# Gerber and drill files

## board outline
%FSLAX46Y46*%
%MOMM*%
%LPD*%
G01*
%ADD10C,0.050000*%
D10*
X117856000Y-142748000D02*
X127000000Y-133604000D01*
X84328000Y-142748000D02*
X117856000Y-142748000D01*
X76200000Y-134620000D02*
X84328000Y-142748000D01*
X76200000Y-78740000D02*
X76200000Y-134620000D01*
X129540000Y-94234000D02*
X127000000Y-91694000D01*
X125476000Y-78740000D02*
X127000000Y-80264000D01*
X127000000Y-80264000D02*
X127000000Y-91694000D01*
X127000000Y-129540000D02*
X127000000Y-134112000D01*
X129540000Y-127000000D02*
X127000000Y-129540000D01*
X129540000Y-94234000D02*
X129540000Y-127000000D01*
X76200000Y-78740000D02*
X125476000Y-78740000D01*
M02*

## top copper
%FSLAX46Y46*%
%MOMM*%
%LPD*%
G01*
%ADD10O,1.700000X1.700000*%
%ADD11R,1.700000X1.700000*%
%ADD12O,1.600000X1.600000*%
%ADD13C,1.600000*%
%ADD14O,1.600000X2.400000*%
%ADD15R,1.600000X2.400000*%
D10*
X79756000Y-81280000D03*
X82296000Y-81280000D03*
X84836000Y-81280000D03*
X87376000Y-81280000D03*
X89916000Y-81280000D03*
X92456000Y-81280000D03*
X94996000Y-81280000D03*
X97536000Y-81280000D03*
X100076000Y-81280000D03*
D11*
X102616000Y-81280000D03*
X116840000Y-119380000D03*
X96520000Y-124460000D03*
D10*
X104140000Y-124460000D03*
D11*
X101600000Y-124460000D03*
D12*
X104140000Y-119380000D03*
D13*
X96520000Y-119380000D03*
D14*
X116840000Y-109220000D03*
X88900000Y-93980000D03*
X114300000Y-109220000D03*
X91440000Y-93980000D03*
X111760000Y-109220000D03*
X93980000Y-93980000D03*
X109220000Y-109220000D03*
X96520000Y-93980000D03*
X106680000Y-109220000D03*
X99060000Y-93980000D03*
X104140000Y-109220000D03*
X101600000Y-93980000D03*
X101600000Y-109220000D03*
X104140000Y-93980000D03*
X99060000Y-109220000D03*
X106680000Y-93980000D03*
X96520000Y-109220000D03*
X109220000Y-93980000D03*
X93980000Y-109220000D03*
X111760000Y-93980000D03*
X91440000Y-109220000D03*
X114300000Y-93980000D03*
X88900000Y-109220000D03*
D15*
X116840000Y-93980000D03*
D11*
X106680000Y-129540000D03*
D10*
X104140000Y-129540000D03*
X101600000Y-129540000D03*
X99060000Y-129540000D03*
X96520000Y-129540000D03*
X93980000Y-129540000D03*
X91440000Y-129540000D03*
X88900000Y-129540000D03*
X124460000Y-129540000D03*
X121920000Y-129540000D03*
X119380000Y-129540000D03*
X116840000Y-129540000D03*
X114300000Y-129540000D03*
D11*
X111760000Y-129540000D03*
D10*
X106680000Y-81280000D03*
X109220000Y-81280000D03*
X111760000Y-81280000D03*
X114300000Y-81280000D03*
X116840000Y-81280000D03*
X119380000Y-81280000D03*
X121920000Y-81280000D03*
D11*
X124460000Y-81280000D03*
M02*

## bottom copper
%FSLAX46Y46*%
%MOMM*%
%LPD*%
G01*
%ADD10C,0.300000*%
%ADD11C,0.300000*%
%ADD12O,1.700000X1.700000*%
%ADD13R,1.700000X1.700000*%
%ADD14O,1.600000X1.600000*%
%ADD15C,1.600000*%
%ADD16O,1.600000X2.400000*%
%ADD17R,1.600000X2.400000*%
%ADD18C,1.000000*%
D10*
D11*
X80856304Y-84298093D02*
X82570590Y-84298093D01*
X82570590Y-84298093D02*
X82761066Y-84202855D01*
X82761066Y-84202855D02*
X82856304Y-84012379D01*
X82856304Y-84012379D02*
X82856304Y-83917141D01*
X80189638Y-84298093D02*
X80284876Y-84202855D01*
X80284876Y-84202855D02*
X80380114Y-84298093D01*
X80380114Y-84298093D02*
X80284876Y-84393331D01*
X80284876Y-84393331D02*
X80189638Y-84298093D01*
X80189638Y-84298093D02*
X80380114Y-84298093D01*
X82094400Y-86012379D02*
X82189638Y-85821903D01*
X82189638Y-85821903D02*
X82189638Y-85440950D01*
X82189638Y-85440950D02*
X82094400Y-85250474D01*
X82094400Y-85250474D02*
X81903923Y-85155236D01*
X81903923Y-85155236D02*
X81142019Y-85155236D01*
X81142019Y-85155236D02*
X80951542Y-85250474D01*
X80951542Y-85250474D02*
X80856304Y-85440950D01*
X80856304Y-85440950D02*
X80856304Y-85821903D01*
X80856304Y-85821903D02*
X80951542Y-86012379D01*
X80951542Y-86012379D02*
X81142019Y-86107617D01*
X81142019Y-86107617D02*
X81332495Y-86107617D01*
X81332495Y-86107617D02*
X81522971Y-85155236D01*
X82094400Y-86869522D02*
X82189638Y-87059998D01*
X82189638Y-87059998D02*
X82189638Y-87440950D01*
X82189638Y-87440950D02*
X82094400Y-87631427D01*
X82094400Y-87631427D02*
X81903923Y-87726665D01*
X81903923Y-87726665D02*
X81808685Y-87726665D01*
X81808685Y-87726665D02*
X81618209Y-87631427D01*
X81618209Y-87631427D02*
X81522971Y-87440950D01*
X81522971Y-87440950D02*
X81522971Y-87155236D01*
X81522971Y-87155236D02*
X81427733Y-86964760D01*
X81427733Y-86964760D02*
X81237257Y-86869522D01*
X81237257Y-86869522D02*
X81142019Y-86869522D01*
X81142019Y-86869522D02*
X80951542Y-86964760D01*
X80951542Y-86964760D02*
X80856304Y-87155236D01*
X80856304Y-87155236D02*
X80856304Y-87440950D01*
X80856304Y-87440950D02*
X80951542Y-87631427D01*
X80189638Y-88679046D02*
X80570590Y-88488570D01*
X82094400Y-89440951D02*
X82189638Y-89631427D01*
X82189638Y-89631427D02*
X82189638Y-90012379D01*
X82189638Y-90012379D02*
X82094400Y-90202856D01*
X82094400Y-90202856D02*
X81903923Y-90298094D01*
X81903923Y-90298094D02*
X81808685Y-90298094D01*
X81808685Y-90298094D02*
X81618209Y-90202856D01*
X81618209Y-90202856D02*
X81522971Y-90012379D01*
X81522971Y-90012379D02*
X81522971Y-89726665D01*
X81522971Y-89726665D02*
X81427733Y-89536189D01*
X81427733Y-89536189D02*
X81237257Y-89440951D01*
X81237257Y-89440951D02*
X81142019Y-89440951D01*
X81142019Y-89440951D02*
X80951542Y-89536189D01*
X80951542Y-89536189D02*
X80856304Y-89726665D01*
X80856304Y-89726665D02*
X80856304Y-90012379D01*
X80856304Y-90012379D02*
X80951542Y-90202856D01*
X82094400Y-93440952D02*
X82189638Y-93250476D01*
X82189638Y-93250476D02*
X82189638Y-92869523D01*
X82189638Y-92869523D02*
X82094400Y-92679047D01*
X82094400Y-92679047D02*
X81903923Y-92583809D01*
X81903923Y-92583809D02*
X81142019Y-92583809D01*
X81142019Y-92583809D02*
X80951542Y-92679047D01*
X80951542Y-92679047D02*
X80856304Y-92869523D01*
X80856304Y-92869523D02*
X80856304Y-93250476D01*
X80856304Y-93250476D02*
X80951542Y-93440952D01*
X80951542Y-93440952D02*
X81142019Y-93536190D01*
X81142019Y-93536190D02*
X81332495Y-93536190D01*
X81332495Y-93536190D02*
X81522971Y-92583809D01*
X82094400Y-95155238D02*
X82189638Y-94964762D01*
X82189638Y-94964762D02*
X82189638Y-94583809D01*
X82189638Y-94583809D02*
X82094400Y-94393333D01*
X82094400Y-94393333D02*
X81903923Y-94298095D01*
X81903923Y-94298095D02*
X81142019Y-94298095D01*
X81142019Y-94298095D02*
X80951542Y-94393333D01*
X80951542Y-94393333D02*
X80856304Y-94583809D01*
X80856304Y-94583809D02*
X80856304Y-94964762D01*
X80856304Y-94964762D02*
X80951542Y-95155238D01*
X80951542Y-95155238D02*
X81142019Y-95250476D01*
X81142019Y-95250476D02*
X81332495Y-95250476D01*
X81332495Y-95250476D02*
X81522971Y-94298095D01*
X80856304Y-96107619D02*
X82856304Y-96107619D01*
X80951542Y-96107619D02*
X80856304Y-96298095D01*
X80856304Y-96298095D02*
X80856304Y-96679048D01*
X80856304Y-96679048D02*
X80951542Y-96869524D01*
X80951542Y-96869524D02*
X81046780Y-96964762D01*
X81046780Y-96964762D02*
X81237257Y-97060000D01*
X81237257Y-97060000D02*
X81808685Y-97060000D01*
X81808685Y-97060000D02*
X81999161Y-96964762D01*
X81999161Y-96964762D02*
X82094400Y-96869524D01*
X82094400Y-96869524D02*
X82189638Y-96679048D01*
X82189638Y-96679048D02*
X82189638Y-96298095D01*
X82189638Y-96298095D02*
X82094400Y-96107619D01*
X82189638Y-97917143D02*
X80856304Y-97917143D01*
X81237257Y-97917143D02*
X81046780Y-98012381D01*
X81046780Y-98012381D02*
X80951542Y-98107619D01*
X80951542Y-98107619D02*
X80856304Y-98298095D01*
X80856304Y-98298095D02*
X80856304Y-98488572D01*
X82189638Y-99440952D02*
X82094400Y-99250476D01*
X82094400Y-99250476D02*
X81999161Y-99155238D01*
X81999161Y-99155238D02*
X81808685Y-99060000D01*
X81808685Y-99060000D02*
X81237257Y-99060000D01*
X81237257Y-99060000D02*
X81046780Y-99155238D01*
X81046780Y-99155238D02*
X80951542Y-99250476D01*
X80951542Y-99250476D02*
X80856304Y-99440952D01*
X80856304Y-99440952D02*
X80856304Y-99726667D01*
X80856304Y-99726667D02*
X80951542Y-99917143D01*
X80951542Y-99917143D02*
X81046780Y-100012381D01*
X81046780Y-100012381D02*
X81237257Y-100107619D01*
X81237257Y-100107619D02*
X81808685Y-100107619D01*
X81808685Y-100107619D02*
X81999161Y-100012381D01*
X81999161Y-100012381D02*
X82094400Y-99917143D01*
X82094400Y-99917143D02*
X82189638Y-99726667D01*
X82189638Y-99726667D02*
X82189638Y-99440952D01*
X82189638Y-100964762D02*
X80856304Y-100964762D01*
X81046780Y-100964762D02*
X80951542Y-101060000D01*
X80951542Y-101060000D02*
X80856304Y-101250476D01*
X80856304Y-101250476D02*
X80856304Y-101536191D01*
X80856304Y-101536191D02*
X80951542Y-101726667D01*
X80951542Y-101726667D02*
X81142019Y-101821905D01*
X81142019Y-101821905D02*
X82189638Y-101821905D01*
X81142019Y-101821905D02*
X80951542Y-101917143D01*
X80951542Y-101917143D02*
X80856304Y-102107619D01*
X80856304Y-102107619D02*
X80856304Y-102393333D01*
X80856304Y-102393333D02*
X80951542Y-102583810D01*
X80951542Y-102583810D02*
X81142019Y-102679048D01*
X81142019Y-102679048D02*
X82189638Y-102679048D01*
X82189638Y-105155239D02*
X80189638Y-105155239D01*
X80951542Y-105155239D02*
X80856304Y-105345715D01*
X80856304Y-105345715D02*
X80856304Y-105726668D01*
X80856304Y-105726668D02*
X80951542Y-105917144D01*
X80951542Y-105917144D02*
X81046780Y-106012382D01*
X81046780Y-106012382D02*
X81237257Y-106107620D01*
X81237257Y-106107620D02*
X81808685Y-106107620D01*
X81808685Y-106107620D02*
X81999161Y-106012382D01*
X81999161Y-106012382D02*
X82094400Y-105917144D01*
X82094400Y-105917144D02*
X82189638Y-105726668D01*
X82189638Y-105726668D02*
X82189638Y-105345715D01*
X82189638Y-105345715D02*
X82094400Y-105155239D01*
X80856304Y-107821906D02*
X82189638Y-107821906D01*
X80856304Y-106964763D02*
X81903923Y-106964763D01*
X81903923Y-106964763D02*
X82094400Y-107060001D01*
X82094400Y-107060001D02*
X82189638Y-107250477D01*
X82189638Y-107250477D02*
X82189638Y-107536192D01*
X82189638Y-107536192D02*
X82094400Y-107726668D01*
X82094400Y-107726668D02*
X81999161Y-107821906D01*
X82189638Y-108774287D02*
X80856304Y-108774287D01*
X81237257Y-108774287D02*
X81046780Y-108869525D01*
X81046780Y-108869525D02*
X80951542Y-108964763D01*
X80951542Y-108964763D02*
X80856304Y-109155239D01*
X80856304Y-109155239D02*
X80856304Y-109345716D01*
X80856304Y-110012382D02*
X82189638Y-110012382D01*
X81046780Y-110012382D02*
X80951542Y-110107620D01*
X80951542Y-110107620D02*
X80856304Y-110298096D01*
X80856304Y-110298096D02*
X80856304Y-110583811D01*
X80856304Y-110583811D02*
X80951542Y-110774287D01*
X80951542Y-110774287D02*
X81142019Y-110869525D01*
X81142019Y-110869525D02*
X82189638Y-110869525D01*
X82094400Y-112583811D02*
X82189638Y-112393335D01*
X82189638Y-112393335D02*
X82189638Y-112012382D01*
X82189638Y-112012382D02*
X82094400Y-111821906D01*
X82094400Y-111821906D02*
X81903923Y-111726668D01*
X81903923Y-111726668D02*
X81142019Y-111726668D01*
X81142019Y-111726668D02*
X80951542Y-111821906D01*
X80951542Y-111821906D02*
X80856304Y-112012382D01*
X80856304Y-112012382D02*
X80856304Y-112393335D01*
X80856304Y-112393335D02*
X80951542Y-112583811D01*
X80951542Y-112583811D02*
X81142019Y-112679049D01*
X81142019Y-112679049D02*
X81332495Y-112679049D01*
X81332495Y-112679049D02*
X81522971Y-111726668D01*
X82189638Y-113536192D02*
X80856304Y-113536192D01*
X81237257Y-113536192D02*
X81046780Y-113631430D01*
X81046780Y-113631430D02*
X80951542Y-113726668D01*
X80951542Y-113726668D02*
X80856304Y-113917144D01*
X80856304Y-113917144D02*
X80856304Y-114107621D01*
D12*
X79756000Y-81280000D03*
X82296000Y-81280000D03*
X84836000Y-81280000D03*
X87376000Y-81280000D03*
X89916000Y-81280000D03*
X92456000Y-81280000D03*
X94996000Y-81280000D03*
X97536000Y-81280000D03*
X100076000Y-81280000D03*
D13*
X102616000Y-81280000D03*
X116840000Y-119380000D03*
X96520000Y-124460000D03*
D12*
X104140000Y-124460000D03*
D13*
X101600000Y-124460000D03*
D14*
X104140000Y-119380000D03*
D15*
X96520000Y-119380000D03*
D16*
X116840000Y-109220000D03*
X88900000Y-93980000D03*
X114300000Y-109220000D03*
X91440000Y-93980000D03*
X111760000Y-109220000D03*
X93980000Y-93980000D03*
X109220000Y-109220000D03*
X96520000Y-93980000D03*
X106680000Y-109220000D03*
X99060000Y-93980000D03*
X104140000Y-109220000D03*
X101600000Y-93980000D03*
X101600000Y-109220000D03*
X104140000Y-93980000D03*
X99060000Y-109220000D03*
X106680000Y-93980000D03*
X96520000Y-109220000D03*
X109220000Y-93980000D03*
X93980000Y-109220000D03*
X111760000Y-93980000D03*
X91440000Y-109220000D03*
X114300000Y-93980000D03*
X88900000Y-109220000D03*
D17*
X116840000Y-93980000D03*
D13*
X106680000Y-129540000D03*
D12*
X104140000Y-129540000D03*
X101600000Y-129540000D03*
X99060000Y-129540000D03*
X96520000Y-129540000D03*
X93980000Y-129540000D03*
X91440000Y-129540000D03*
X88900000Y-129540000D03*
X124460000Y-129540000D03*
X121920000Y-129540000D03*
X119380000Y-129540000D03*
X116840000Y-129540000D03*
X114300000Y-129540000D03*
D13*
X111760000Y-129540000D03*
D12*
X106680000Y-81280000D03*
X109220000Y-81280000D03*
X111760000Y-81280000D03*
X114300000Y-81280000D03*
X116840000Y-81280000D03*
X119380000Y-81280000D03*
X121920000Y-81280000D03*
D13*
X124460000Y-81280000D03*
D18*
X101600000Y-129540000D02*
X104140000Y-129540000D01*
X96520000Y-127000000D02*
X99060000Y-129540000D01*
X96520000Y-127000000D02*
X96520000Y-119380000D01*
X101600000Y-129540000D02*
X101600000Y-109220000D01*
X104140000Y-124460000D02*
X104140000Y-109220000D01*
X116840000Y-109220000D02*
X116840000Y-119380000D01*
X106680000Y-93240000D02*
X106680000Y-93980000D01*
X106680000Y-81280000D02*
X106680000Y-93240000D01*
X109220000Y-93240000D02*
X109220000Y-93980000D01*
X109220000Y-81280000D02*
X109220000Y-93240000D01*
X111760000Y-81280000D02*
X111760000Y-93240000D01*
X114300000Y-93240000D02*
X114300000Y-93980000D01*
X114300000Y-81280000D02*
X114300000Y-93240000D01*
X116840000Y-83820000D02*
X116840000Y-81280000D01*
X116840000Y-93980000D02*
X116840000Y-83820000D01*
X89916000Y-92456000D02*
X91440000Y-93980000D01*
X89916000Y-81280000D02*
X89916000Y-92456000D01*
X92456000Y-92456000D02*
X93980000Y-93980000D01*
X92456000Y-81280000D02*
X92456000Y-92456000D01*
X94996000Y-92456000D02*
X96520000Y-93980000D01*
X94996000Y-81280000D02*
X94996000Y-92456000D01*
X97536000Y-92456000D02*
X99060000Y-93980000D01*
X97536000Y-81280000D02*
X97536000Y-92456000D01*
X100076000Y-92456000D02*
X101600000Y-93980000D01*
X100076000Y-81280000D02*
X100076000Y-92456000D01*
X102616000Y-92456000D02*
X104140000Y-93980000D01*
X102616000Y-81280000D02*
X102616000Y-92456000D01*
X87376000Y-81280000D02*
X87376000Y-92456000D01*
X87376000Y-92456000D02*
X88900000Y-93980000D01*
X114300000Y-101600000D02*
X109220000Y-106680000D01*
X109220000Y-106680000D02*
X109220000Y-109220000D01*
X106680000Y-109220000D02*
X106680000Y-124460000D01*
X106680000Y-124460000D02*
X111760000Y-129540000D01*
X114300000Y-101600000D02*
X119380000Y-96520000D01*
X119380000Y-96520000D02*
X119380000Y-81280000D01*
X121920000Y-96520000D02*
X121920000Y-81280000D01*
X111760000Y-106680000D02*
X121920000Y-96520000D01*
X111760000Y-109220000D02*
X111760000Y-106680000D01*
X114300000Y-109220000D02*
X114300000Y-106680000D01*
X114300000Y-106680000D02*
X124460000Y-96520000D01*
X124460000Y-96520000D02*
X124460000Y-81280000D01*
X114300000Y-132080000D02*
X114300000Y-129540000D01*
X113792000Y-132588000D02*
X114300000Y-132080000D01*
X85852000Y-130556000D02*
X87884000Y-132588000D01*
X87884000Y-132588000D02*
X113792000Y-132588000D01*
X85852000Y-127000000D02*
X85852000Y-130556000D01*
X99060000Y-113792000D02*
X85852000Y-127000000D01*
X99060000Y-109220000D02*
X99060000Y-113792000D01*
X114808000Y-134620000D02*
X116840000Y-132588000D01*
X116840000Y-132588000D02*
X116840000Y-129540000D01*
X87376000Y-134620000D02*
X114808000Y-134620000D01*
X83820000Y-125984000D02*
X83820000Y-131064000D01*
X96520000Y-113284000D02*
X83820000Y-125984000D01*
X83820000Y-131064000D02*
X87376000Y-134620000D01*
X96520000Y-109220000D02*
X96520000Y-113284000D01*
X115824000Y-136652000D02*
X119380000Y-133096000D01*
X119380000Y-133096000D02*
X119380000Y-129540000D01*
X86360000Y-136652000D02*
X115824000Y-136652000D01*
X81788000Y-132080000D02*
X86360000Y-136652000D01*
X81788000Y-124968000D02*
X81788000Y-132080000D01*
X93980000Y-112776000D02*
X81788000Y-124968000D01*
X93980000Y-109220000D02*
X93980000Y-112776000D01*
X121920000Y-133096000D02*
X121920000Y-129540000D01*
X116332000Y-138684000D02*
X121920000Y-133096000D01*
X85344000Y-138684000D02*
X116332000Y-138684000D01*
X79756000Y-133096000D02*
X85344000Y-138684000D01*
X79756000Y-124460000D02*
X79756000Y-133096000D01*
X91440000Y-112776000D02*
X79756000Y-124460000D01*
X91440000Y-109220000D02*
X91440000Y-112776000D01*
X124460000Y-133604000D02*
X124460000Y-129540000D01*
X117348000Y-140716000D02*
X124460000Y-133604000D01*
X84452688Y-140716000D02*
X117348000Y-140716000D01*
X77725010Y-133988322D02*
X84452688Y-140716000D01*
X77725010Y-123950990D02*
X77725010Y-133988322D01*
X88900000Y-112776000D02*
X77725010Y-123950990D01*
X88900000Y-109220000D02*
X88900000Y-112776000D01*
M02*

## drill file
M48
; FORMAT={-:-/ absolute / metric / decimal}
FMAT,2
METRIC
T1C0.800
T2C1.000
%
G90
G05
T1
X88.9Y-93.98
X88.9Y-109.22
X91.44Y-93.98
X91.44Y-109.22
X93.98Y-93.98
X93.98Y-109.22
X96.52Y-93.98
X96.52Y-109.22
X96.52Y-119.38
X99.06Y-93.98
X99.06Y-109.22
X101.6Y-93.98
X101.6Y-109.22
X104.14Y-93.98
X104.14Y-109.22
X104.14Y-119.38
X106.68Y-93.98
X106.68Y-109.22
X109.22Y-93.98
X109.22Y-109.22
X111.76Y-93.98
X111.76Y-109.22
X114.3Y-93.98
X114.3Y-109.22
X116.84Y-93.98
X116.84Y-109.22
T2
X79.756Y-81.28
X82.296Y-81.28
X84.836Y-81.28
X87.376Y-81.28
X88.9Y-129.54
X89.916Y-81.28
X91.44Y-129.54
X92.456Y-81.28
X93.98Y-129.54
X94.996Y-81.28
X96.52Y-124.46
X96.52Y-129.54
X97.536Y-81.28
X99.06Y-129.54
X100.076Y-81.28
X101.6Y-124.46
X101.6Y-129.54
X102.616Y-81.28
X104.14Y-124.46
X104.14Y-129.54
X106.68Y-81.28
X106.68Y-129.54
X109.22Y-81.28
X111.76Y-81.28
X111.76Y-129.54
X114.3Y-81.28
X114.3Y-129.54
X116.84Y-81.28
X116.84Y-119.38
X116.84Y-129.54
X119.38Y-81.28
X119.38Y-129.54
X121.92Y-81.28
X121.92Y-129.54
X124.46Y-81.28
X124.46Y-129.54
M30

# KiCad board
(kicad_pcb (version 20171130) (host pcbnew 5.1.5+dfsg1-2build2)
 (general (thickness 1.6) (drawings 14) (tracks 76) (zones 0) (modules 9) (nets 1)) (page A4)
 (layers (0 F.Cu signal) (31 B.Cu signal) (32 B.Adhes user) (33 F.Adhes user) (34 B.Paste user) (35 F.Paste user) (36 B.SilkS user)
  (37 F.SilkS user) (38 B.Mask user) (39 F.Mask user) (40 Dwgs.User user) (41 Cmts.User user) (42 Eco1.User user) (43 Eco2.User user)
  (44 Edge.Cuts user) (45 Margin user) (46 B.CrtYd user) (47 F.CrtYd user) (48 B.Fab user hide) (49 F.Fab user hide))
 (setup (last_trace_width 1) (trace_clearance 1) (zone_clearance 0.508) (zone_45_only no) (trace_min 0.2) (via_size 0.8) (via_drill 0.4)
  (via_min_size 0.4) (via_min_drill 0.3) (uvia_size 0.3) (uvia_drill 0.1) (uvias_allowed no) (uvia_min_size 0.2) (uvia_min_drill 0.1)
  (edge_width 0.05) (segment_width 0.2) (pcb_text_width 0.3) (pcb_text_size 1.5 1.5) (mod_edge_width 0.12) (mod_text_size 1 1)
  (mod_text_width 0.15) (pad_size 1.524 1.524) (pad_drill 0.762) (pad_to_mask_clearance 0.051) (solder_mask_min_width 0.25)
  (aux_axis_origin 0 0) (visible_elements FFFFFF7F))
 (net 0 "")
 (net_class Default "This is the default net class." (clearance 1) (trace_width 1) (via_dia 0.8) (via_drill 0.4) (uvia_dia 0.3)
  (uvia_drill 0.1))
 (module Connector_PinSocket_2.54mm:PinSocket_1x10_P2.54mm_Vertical (layer F.Cu) (at 102.616 81.28 270)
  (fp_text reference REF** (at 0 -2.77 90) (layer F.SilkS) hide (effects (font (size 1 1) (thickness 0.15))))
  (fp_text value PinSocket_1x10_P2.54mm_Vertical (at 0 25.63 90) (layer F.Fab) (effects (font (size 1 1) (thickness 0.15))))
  (pad 10 thru_hole oval (at 0 22.86 270) (size 1.7 1.7) (drill 1) (layers *.Cu *.Mask))
  (pad 9 thru_hole oval (at 0 20.32 270) (size 1.7 1.7) (drill 1) (layers *.Cu *.Mask))
  (pad 8 thru_hole oval (at 0 17.78 270) (size 1.7 1.7) (drill 1) (layers *.Cu *.Mask))
  (pad 7 thru_hole oval (at 0 15.24 270) (size 1.7 1.7) (drill 1) (layers *.Cu *.Mask))
  (pad 6 thru_hole oval (at 0 12.7 270) (size 1.7 1.7) (drill 1) (layers *.Cu *.Mask))
  (pad 5 thru_hole oval (at 0 10.16 270) (size 1.7 1.7) (drill 1) (layers *.Cu *.Mask))
  (pad 4 thru_hole oval (at 0 7.62 270) (size 1.7 1.7) (drill 1) (layers *.Cu *.Mask))
  (pad 3 thru_hole oval (at 0 5.08 270) (size 1.7 1.7) (drill 1) (layers *.Cu *.Mask))
  (pad 2 thru_hole oval (at 0 2.54 270) (size 1.7 1.7) (drill 1) (layers *.Cu *.Mask))
  (pad 1 thru_hole rect (at 0 0 270) (size 1.7 1.7) (drill 1) (layers *.Cu *.Mask)))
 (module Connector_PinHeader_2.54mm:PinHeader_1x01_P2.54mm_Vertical (layer F.Cu) (at 116.84 119.38)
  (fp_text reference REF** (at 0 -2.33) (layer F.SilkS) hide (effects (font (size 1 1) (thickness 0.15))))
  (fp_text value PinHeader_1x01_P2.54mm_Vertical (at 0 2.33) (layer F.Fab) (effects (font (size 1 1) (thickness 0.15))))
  (pad 1 thru_hole rect (at 0 0) (size 1.7 1.7) (drill 1) (layers *.Cu *.Mask)))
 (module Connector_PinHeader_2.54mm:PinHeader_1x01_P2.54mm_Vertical (layer F.Cu) (at 96.52 124.46)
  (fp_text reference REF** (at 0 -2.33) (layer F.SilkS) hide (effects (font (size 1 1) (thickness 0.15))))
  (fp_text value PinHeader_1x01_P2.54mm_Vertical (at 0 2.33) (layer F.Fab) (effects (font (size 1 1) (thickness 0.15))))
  (pad 1 thru_hole rect (at 0 0) (size 1.7 1.7) (drill 1) (layers *.Cu *.Mask)))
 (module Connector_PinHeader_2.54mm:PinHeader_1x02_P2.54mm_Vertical (layer F.Cu) (at 101.6 124.46 90)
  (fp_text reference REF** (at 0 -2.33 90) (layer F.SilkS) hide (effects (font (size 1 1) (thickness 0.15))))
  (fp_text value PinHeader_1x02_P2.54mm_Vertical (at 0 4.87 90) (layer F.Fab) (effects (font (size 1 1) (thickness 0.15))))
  (pad 2 thru_hole oval (at 0 2.54 90) (size 1.7 1.7) (drill 1) (layers *.Cu *.Mask))
  (pad 1 thru_hole rect (at 0 0 90) (size 1.7 1.7) (drill 1) (layers *.Cu *.Mask)))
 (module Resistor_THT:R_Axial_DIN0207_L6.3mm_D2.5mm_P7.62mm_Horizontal (layer F.Cu) (at 96.52 119.38)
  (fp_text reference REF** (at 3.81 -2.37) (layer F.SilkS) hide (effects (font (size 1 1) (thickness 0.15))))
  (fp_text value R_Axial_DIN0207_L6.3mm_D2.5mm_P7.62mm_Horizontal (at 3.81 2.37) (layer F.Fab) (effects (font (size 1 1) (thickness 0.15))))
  (pad 2 thru_hole oval (at 7.62 0) (size 1.6 1.6) (drill 0.8) (layers *.Cu *.Mask))
  (pad 1 thru_hole circle (at 0 0) (size 1.6 1.6) (drill 0.8) (layers *.Cu *.Mask)))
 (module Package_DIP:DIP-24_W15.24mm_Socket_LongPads (layer F.Cu) (at 116.84 93.98 270)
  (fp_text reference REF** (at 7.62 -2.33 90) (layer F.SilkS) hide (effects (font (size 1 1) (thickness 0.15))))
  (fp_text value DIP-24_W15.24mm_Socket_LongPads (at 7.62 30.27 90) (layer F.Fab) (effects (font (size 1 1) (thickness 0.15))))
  (pad 24 thru_hole oval (at 15.24 0 270) (size 2.4 1.6) (drill 0.8) (layers *.Cu *.Mask))
  (pad 12 thru_hole oval (at 0 27.94 270) (size 2.4 1.6) (drill 0.8) (layers *.Cu *.Mask))
  (pad 23 thru_hole oval (at 15.24 2.54 270) (size 2.4 1.6) (drill 0.8) (layers *.Cu *.Mask))
  (pad 11 thru_hole oval (at 0 25.4 270) (size 2.4 1.6) (drill 0.8) (layers *.Cu *.Mask))
  (pad 22 thru_hole oval (at 15.24 5.08 270) (size 2.4 1.6) (drill 0.8) (layers *.Cu *.Mask))
  (pad 10 thru_hole oval (at 0 22.86 270) (size 2.4 1.6) (drill 0.8) (layers *.Cu *.Mask))
  (pad 21 thru_hole oval (at 15.24 7.62 270) (size 2.4 1.6) (drill 0.8) (layers *.Cu *.Mask))
  (pad 9 thru_hole oval (at 0 20.32 270) (size 2.4 1.6) (drill 0.8) (layers *.Cu *.Mask))
  (pad 20 thru_hole oval (at 15.24 10.16 270) (size 2.4 1.6) (drill 0.8) (layers *.Cu *.Mask))
  (pad 8 thru_hole oval (at 0 17.78 270) (size 2.4 1.6) (drill 0.8) (layers *.Cu *.Mask))
  (pad 19 thru_hole oval (at 15.24 12.7 270) (size 2.4 1.6) (drill 0.8) (layers *.Cu *.Mask))
  (pad 7 thru_hole oval (at 0 15.24 270) (size 2.4 1.6) (drill 0.8) (layers *.Cu *.Mask))
  (pad 18 thru_hole oval (at 15.24 15.24 270) (size 2.4 1.6) (drill 0.8) (layers *.Cu *.Mask))
  (pad 6 thru_hole oval (at 0 12.7 270) (size 2.4 1.6) (drill 0.8) (layers *.Cu *.Mask))
  (pad 17 thru_hole oval (at 15.24 17.78 270) (size 2.4 1.6) (drill 0.8) (layers *.Cu *.Mask))
  (pad 5 thru_hole oval (at 0 10.16 270) (size 2.4 1.6) (drill 0.8) (layers *.Cu *.Mask))
  (pad 16 thru_hole oval (at 15.24 20.32 270) (size 2.4 1.6) (drill 0.8) (layers *.Cu *.Mask))
  (pad 4 thru_hole oval (at 0 7.62 270) (size 2.4 1.6) (drill 0.8) (layers *.Cu *.Mask))
  (pad 15 thru_hole oval (at 15.24 22.86 270) (size 2.4 1.6) (drill 0.8) (layers *.Cu *.Mask))
  (pad 3 thru_hole oval (at 0 5.08 270) (size 2.4 1.6) (drill 0.8) (layers *.Cu *.Mask))
  (pad 14 thru_hole oval (at 15.24 25.4 270) (size 2.4 1.6) (drill 0.8) (layers *.Cu *.Mask))
  (pad 2 thru_hole oval (at 0 2.54 270) (size 2.4 1.6) (drill 0.8) (layers *.Cu *.Mask))
  (pad 13 thru_hole oval (at 15.24 27.94 270) (size 2.4 1.6) (drill 0.8) (layers *.Cu *.Mask))
  (pad 1 thru_hole rect (at 0 0 270) (size 2.4 1.6) (drill 0.8) (layers *.Cu *.Mask)))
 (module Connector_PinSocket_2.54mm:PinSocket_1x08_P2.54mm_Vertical (layer F.Cu) (at 106.68 129.54 270)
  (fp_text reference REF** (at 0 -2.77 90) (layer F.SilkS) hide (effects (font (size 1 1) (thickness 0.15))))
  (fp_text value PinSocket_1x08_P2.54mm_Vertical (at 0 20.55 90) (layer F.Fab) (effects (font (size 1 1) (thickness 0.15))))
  (pad 1 thru_hole rect (at 0 0 270) (size 1.7 1.7) (drill 1) (layers *.Cu *.Mask))
  (pad 2 thru_hole oval (at 0 2.54 270) (size 1.7 1.7) (drill 1) (layers *.Cu *.Mask))
  (pad 3 thru_hole oval (at 0 5.08 270) (size 1.7 1.7) (drill 1) (layers *.Cu *.Mask))
  (pad 4 thru_hole oval (at 0 7.62 270) (size 1.7 1.7) (drill 1) (layers *.Cu *.Mask))
  (pad 5 thru_hole oval (at 0 10.16 270) (size 1.7 1.7) (drill 1) (layers *.Cu *.Mask))
  (pad 6 thru_hole oval (at 0 12.7 270) (size 1.7 1.7) (drill 1) (layers *.Cu *.Mask))
  (pad 7 thru_hole oval (at 0 15.24 270) (size 1.7 1.7) (drill 1) (layers *.Cu *.Mask))
  (pad 8 thru_hole oval (at 0 17.78 270) (size 1.7 1.7) (drill 1) (layers *.Cu *.Mask)))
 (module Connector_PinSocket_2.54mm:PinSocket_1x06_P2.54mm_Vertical (layer F.Cu) (at 111.76 129.54 90)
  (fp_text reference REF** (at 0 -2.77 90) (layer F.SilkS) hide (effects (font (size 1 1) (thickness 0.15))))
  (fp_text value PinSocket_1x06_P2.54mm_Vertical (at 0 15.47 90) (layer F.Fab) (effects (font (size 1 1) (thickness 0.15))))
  (pad 6 thru_hole oval (at 0 12.7 90) (size 1.7 1.7) (drill 1) (layers *.Cu *.Mask))
  (pad 5 thru_hole oval (at 0 10.16 90) (size 1.7 1.7) (drill 1) (layers *.Cu *.Mask))
  (pad 4 thru_hole oval (at 0 7.62 90) (size 1.7 1.7) (drill 1) (layers *.Cu *.Mask))
  (pad 3 thru_hole oval (at 0 5.08 90) (size 1.7 1.7) (drill 1) (layers *.Cu *.Mask))
  (pad 2 thru_hole oval (at 0 2.54 90) (size 1.7 1.7) (drill 1) (layers *.Cu *.Mask))
  (pad 1 thru_hole rect (at 0 0 90) (size 1.7 1.7) (drill 1) (layers *.Cu *.Mask)))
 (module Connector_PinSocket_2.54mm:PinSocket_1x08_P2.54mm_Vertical (layer F.Cu) (at 124.46 81.28 270)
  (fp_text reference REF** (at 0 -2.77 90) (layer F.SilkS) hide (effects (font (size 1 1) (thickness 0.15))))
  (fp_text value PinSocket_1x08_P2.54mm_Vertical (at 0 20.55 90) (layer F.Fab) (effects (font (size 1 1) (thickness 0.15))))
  (pad 8 thru_hole oval (at 0 17.78 270) (size 1.7 1.7) (drill 1) (layers *.Cu *.Mask))
  (pad 7 thru_hole oval (at 0 15.24 270) (size 1.7 1.7) (drill 1) (layers *.Cu *.Mask))
  (pad 6 thru_hole oval (at 0 12.7 270) (size 1.7 1.7) (drill 1) (layers *.Cu *.Mask))
  (pad 5 thru_hole oval (at 0 10.16 270) (size 1.7 1.7) (drill 1) (layers *.Cu *.Mask))
  (pad 4 thru_hole oval (at 0 7.62 270) (size 1.7 1.7) (drill 1) (layers *.Cu *.Mask))
  (pad 3 thru_hole oval (at 0 5.08 270) (size 1.7 1.7) (drill 1) (layers *.Cu *.Mask))
  (pad 2 thru_hole oval (at 0 2.54 270) (size 1.7 1.7) (drill 1) (layers *.Cu *.Mask))
  (pad 1 thru_hole rect (at 0 0 270) (size 1.7 1.7) (drill 1) (layers *.Cu *.Mask)))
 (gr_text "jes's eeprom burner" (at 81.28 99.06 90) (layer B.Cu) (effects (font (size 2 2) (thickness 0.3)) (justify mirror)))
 (gr_line (start 117.856 142.748) (end 127 133.604) (layer Edge.Cuts) (width 0.05))
 (gr_line (start 84.328 142.748) (end 117.856 142.748) (layer Edge.Cuts) (width 0.05))
 (gr_line (start 76.2 134.62) (end 84.328 142.748) (layer Edge.Cuts) (width 0.05))
 (gr_line (start 76.2 78.74) (end 76.2 134.62) (layer Edge.Cuts) (width 0.05))
 (gr_line (start 129.54 94.234) (end 127 91.694) (layer Edge.Cuts) (width 0.05))
 (gr_line (start 125.476 78.74) (end 127 80.264) (layer Edge.Cuts) (width 0.05))
 (gr_line (start 127 80.264) (end 127 91.694) (layer Edge.Cuts) (width 0.05))
 (gr_line (start 127 129.54) (end 127 134.112) (layer Edge.Cuts) (width 0.05))
 (gr_line (start 129.54 127) (end 127 129.54) (layer Edge.Cuts) (width 0.05))
 (gr_line (start 129.54 94.234) (end 129.54 127) (layer Edge.Cuts) (width 0.05))
 (gr_line (start 76.2 78.74) (end 125.476 78.74) (layer Edge.Cuts) (width 0.05))
 (segment (start 101.6 129.54) (end 104.14 129.54) (width 1) (layer B.Cu) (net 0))
 (segment (start 96.52 127) (end 99.06 129.54) (width 1) (layer B.Cu) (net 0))
 (segment (start 96.52 127) (end 96.52 119.38) (width 1) (layer B.Cu) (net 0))
 (segment (start 101.6 129.54) (end 101.6 109.22) (width 1) (layer B.Cu) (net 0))
 (segment (start 104.14 124.46) (end 104.14 109.22) (width 1) (layer B.Cu) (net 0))
 (segment (start 116.84 109.22) (end 116.84 119.38) (width 1) (layer B.Cu) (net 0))
 (segment (start 106.68 93.24) (end 106.68 93.98) (width 1) (layer B.Cu) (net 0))
 (segment (start 106.68 81.28) (end 106.68 93.24) (width 1) (layer B.Cu) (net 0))
 (segment (start 109.22 93.24) (end 109.22 93.98) (width 1) (layer B.Cu) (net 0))
 (segment (start 109.22 81.28) (end 109.22 93.24) (width 1) (layer B.Cu) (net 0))
 (segment (start 111.76 81.28) (end 111.76 93.24) (width 1) (layer B.Cu) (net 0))
 (segment (start 114.3 93.24) (end 114.3 93.98) (width 1) (layer B.Cu) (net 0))
 (segment (start 114.3 81.28) (end 114.3 93.24) (width 1) (layer B.Cu) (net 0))
 (segment (start 116.84 83.82) (end 116.84 81.28) (width 1) (layer B.Cu) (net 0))
 (segment (start 116.84 93.98) (end 116.84 83.82) (width 1) (layer B.Cu) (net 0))
 (segment (start 89.916 92.456) (end 91.44 93.98) (width 1) (layer B.Cu) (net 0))
 (segment (start 89.916 81.28) (end 89.916 92.456) (width 1) (layer B.Cu) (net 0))
 (segment (start 92.456 92.456) (end 93.98 93.98) (width 1) (layer B.Cu) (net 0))
 (segment (start 92.456 81.28) (end 92.456 92.456) (width 1) (layer B.Cu) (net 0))
 (segment (start 94.996 92.456) (end 96.52 93.98) (width 1) (layer B.Cu) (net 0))
 (segment (start 94.996 81.28) (end 94.996 92.456) (width 1) (layer B.Cu) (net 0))
 (segment (start 97.536 92.456) (end 99.06 93.98) (width 1) (layer B.Cu) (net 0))
 (segment (start 97.536 81.28) (end 97.536 92.456) (width 1) (layer B.Cu) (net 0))
 (segment (start 100.076 92.456) (end 101.6 93.98) (width 1) (layer B.Cu) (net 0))
 (segment (start 100.076 81.28) (end 100.076 92.456) (width 1) (layer B.Cu) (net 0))
 (segment (start 102.616 92.456) (end 104.14 93.98) (width 1) (layer B.Cu) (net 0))
 (segment (start 102.616 81.28) (end 102.616 92.456) (width 1) (layer B.Cu) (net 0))
 (segment (start 87.376 81.28) (end 87.376 92.456) (width 1) (layer B.Cu) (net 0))
 (segment (start 87.376 92.456) (end 88.9 93.98) (width 1) (layer B.Cu) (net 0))
 (segment (start 114.3 101.6) (end 109.22 106.68) (width 1) (layer B.Cu) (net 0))
 (segment (start 109.22 106.68) (end 109.22 109.22) (width 1) (layer B.Cu) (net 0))
 (segment (start 106.68 109.22) (end 106.68 124.46) (width 1) (layer B.Cu) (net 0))
 (segment (start 106.68 124.46) (end 111.76 129.54) (width 1) (layer B.Cu) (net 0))
 (segment (start 114.3 101.6) (end 119.38 96.52) (width 1) (layer B.Cu) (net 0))
 (segment (start 119.38 96.52) (end 119.38 81.28) (width 1) (layer B.Cu) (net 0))
 (segment (start 121.92 96.52) (end 121.92 81.28) (width 1) (layer B.Cu) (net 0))
 (segment (start 111.76 106.68) (end 121.92 96.52) (width 1) (layer B.Cu) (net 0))
 (segment (start 111.76 109.22) (end 111.76 106.68) (width 1) (layer B.Cu) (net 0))
 (segment (start 114.3 109.22) (end 114.3 106.68) (width 1) (layer B.Cu) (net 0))
 (segment (start 114.3 106.68) (end 124.46 96.52) (width 1) (layer B.Cu) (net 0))
 (segment (start 124.46 96.52) (end 124.46 81.28) (width 1) (layer B.Cu) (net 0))
 (segment (start 114.3 132.08) (end 114.3 129.54) (width 1) (layer B.Cu) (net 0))
 (segment (start 113.792 132.588) (end 114.3 132.08) (width 1) (layer B.Cu) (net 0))
 (segment (start 85.852 130.556) (end 87.884 132.588) (width 1) (layer B.Cu) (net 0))
 (segment (start 87.884 132.588) (end 113.792 132.588) (width 1) (layer B.Cu) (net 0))
 (segment (start 85.852 127) (end 85.852 130.556) (width 1) (layer B.Cu) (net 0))
 (segment (start 99.06 113.792) (end 85.852 127) (width 1) (layer B.Cu) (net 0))
 (segment (start 99.06 109.22) (end 99.06 113.792) (width 1) (layer B.Cu) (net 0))
 (segment (start 114.808 134.62) (end 116.84 132.588) (width 1) (layer B.Cu) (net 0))
 (segment (start 116.84 132.588) (end 116.84 129.54) (width 1) (layer B.Cu) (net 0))
 (segment (start 87.376 134.62) (end 114.808 134.62) (width 1) (layer B.Cu) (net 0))
 (segment (start 83.82 125.984) (end 83.82 131.064) (width 1) (layer B.Cu) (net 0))
 (segment (start 96.52 113.284) (end 83.82 125.984) (width 1) (layer B.Cu) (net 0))
 (segment (start 83.82 131.064) (end 87.376 134.62) (width 1) (layer B.Cu) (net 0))
 (segment (start 96.52 109.22) (end 96.52 113.284) (width 1) (layer B.Cu) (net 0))
 (segment (start 115.824 136.652) (end 119.38 133.096) (width 1) (layer B.Cu) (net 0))
 (segment (start 119.38 133.096) (end 119.38 129.54) (width 1) (layer B.Cu) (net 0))
 (segment (start 86.36 136.652) (end 115.824 136.652) (width 1) (layer B.Cu) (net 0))
 (segment (start 81.788 132.08) (end 86.36 136.652) (width 1) (layer B.Cu) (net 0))
 (segment (start 81.788 124.968) (end 81.788 132.08) (width 1) (layer B.Cu) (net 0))
 (segment (start 93.98 112.776) (end 81.788 124.968) (width 1) (layer B.Cu) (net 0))
 (segment (start 93.98 109.22) (end 93.98 112.776) (width 1) (layer B.Cu) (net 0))
 (segment (start 121.92 133.096) (end 121.92 129.54) (width 1) (layer B.Cu) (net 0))
 (segment (start 116.332 138.684) (end 121.92 133.096) (width 1) (layer B.Cu) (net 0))
 (segment (start 85.344 138.684) (end 116.332 138.684) (width 1) (layer B.Cu) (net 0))
 (segment (start 79.756 133.096) (end 85.344 138.684) (width 1) (layer B.Cu) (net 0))
 (segment (start 79.756 124.46) (end 79.756 133.096) (width 1) (layer B.Cu) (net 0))
 (segment (start 91.44 112.776) (end 79.756 124.46) (width 1) (layer B.Cu) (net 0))
 (segment (start 91.44 109.22) (end 91.44 112.776) (width 1) (layer B.Cu) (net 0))
 (segment (start 124.46 133.604) (end 124.46 129.54) (width 1) (layer B.Cu) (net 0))
 (segment (start 117.348 140.716) (end 124.46 133.604) (width 1) (layer B.Cu) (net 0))
 (segment (start 84.452688 140.716) (end 117.348 140.716) (width 1) (layer B.Cu) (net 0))
 (segment (start 77.72501 133.988322) (end 84.452688 140.716) (width 1) (layer B.Cu) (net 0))
 (segment (start 77.72501 123.95099) (end 77.72501 133.988322) (width 1) (layer B.Cu) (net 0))
 (segment (start 88.9 112.776) (end 77.72501 123.95099) (width 1) (layer B.Cu) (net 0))
 (segment (start 88.9 109.22) (end 88.9 112.776) (width 1) (layer B.Cu) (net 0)))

